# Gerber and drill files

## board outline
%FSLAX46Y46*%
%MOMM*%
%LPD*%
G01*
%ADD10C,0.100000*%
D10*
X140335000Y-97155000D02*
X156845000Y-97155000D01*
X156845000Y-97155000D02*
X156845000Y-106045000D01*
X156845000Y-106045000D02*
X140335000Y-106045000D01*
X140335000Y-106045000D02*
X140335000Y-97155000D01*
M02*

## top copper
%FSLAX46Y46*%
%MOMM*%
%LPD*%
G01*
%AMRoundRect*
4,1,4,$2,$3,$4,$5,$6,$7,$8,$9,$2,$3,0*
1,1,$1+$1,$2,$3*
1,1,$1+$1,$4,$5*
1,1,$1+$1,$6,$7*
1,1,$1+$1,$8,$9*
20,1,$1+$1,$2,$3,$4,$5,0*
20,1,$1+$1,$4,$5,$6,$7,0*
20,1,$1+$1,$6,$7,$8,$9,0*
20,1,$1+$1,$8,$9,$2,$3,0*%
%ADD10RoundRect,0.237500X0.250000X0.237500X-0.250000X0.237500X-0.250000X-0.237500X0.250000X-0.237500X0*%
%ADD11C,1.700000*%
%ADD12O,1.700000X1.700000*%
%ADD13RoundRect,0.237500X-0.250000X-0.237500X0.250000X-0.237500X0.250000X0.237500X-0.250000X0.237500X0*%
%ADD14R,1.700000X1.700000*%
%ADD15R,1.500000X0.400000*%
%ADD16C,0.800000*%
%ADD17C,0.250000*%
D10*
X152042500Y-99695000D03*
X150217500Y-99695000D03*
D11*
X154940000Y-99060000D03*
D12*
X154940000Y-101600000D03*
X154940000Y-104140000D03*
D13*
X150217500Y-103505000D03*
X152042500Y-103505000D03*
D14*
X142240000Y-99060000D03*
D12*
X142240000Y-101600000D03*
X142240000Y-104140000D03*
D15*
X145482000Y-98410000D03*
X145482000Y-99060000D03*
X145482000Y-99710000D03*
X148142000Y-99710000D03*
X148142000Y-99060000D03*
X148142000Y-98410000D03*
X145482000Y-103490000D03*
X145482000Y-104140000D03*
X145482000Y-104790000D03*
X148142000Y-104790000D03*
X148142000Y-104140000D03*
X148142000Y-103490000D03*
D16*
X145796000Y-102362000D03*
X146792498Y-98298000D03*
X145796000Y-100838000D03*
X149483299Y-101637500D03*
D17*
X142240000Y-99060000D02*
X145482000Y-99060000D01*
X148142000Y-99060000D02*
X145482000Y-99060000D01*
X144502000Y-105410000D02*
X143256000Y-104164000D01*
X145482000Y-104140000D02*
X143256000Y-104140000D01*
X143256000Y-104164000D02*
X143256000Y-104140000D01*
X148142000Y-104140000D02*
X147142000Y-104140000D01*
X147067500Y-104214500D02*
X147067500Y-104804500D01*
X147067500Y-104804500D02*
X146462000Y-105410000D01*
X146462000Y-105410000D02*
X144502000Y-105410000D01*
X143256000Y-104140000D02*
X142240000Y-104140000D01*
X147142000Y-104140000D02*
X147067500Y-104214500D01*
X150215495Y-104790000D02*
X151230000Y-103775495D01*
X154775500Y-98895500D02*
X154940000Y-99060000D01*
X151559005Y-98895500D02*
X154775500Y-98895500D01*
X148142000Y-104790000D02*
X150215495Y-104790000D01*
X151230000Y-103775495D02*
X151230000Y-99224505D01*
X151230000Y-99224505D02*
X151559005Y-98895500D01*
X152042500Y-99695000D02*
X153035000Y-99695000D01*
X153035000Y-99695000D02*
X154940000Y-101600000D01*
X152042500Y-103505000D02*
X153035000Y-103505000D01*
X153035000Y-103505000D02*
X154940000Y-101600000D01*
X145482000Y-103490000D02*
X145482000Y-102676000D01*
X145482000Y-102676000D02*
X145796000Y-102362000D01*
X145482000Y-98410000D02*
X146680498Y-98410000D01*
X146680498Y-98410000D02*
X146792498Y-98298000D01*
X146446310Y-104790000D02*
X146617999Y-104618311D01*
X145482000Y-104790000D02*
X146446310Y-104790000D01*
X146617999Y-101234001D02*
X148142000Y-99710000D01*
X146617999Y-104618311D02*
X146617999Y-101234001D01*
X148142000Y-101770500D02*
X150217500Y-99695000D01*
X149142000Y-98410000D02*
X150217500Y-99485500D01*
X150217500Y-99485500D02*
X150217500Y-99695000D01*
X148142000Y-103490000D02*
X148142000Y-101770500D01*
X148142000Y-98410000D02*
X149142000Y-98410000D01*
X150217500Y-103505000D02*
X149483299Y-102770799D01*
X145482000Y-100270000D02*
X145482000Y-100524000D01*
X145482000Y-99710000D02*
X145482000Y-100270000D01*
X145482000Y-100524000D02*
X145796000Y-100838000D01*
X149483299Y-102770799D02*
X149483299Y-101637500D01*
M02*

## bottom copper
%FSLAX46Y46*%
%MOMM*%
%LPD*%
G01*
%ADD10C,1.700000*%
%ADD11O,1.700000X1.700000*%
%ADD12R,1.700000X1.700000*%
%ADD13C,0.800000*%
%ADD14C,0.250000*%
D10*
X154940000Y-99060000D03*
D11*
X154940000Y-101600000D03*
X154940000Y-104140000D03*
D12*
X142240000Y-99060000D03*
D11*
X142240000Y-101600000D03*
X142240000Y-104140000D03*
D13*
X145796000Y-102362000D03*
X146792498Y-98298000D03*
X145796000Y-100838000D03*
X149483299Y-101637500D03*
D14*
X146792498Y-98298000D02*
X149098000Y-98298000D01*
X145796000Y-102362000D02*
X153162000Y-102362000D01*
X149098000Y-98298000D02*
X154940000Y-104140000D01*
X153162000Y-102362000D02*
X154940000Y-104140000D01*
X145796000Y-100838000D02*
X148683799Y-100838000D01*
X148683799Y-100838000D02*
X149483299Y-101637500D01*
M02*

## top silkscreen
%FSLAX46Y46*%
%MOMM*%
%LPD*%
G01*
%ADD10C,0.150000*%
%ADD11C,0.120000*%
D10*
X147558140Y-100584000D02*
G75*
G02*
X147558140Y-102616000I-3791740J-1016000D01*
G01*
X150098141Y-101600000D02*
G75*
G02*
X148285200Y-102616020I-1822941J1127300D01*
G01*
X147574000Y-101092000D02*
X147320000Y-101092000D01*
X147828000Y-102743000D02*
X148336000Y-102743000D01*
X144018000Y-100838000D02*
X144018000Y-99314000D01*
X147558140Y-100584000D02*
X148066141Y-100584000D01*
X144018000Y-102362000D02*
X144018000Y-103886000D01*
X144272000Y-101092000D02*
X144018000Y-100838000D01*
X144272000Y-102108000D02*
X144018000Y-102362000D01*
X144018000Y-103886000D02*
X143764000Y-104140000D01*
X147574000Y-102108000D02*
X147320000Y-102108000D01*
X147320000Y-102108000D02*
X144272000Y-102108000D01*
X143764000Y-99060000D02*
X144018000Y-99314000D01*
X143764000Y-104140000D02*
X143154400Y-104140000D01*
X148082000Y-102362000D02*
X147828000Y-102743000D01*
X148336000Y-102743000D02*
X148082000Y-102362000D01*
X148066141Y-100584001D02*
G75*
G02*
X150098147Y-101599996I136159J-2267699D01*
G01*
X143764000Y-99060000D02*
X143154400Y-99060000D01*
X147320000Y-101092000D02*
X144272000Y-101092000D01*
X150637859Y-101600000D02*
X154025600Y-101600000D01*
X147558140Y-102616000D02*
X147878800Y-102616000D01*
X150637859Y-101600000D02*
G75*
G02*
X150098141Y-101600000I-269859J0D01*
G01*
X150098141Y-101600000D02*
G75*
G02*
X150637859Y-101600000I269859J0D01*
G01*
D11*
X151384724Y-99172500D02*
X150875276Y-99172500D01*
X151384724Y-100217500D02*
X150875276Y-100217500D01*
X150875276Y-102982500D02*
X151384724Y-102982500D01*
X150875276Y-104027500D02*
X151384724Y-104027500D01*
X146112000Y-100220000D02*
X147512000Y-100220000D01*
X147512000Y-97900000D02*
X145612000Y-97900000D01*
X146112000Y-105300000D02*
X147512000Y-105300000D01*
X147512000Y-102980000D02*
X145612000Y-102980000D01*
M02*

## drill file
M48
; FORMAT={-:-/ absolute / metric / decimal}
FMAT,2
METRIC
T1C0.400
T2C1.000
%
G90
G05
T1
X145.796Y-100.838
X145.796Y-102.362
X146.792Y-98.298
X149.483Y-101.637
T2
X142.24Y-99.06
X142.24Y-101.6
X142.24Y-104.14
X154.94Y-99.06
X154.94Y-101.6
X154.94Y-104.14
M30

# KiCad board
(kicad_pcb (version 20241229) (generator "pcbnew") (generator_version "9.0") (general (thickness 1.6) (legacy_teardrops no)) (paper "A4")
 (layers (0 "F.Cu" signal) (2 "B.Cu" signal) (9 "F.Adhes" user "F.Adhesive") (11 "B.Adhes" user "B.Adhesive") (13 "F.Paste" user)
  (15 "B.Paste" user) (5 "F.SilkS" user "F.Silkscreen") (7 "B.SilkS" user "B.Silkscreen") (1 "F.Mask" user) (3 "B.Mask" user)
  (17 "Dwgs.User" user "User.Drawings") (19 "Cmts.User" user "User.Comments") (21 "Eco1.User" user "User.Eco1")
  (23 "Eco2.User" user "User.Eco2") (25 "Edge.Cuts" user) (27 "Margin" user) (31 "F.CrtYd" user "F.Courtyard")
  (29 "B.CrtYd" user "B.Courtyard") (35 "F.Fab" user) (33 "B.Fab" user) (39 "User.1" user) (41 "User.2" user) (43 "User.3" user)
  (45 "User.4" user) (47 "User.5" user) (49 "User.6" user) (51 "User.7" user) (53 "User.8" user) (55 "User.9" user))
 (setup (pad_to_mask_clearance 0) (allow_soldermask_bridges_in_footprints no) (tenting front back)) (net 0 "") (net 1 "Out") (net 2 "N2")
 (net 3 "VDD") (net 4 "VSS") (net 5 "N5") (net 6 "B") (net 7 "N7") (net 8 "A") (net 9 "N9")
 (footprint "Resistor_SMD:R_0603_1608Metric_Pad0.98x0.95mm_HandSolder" (layer "F.Cu") (at 151.13 99.695 180)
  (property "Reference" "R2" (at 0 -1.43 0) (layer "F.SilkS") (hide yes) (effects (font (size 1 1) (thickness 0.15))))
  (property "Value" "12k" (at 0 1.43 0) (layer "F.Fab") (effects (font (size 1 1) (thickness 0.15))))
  (fp_line (start -0.254724 0.5225) (end 0.254724 0.5225) (stroke (width 0.12) (type solid)) (layer "F.SilkS"))
  (fp_line (start -0.254724 -0.5225) (end 0.254724 -0.5225) (stroke (width 0.12) (type solid)) (layer "F.SilkS"))
  (pad "1" smd roundrect (at -0.9125 0 180) (size 0.975 0.95) (layers "F.Cu" "F.Mask" "F.Paste") (roundrect_rratio 0.25) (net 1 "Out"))
  (pad "2" smd roundrect (at 0.9125 0 180) (size 0.975 0.95) (layers "F.Cu" "F.Mask" "F.Paste") (roundrect_rratio 0.25) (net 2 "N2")))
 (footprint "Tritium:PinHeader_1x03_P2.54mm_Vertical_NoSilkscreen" (layer "F.Cu") (at 154.94 99.06)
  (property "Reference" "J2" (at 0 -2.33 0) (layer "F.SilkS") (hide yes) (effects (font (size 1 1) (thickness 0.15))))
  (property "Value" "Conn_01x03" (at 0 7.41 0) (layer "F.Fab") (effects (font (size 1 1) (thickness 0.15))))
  (pad "1" thru_hole circle (at 0 0) (size 1.7 1.7) (drill 1) (layers "*.Cu" "*.Mask") (remove_unused_layers no) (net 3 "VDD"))
  (pad "2" thru_hole oval (at 0 2.54) (size 1.7 1.7) (drill 1) (layers "*.Cu" "*.Mask") (remove_unused_layers no) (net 1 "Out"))
  (pad "3" thru_hole oval (at 0 5.08) (size 1.7 1.7) (drill 1) (layers "*.Cu" "*.Mask") (remove_unused_layers no) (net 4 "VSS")))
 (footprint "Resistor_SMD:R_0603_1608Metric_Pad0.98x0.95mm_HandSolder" (layer "F.Cu") (at 151.13 103.505)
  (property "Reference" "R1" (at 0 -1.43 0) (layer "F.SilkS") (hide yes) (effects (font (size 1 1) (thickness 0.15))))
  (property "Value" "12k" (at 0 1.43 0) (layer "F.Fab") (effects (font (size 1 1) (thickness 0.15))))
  (fp_line (start -0.254724 -0.5225) (end 0.254724 -0.5225) (stroke (width 0.12) (type solid)) (layer "F.SilkS"))
  (fp_line (start -0.254724 0.5225) (end 0.254724 0.5225) (stroke (width 0.12) (type solid)) (layer "F.SilkS"))
  (pad "1" smd roundrect (at -0.9125 0) (size 0.975 0.95) (layers "F.Cu" "F.Mask" "F.Paste") (roundrect_rratio 0.25) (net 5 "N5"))
  (pad "2" smd roundrect (at 0.9125 0) (size 0.975 0.95) (layers "F.Cu" "F.Mask" "F.Paste") (roundrect_rratio 0.25) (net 1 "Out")))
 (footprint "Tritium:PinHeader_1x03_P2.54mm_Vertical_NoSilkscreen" (layer "F.Cu") (at 142.24 99.06)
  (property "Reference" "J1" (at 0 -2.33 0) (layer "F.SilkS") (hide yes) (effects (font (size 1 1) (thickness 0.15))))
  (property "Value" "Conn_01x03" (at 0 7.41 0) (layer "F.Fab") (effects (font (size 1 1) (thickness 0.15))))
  (pad "1" thru_hole rect (at 0 0) (size 1.7 1.7) (drill 1) (layers "*.Cu" "*.Mask") (remove_unused_layers no) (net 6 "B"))
  (pad "2" thru_hole oval (at 0 2.54) (size 1.7 1.7) (drill 1) (layers "*.Cu" "*.Mask") (remove_unused_layers no) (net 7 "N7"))
  (pad "3" thru_hole oval (at 0 5.08) (size 1.7 1.7) (drill 1) (layers "*.Cu" "*.Mask") (remove_unused_layers no) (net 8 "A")))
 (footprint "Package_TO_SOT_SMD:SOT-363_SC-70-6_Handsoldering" (layer "F.Cu") (at 146.812 99.06)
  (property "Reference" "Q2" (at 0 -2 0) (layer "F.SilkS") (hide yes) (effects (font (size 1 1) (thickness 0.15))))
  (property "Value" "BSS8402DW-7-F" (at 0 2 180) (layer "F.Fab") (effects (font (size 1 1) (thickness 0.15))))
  (fp_line (start -0.7 1.16) (end 0.7 1.16) (stroke (width 0.12) (type solid)) (layer "F.SilkS"))
  (fp_line (start 0.7 -1.16) (end -1.2 -1.16) (stroke (width 0.12) (type solid)) (layer "F.SilkS"))
  (pad "1" smd rect (at -1.33 -0.65) (size 1.5 0.4) (layers "F.Cu" "F.Mask" "F.Paste") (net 4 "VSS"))
  (pad "2" smd rect (at -1.33 0) (size 1.5 0.4) (layers "F.Cu" "F.Mask" "F.Paste") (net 6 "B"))
  (pad "3" smd rect (at -1.33 0.65) (size 1.5 0.4) (layers "F.Cu" "F.Mask" "F.Paste") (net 5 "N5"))
  (pad "4" smd rect (at 1.33 0.65) (size 1.5 0.4) (layers "F.Cu" "F.Mask" "F.Paste") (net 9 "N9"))
  (pad "5" smd rect (at 1.33 0) (size 1.5 0.4) (layers "F.Cu" "F.Mask" "F.Paste") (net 6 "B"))
  (pad "6" smd rect (at 1.33 -0.65) (size 1.5 0.4) (layers "F.Cu" "F.Mask" "F.Paste") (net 2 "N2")))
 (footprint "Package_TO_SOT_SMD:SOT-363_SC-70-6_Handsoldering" (layer "F.Cu") (at 146.812 104.14)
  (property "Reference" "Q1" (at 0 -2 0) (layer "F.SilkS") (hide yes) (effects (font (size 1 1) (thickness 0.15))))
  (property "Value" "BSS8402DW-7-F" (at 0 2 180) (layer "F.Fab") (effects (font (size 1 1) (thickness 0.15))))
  (fp_line (start -0.7 1.16) (end 0.7 1.16) (stroke (width 0.12) (type solid)) (layer "F.SilkS"))
  (fp_line (start 0.7 -1.16) (end -1.2 -1.16) (stroke (width 0.12) (type solid)) (layer "F.SilkS"))
  (pad "1" smd rect (at -1.33 -0.65) (size 1.5 0.4) (layers "F.Cu" "F.Mask" "F.Paste") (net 4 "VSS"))
  (pad "2" smd rect (at -1.33 0) (size 1.5 0.4) (layers "F.Cu" "F.Mask" "F.Paste") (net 8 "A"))
  (pad "3" smd rect (at -1.33 0.65) (size 1.5 0.4) (layers "F.Cu" "F.Mask" "F.Paste") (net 9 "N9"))
  (pad "4" smd rect (at 1.33 0.65) (size 1.5 0.4) (layers "F.Cu" "F.Mask" "F.Paste") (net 3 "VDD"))
  (pad "5" smd rect (at 1.33 0) (size 1.5 0.4) (layers "F.Cu" "F.Mask" "F.Paste") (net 8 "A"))
  (pad "6" smd rect (at 1.33 -0.65) (size 1.5 0.4) (layers "F.Cu" "F.Mask" "F.Paste") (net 2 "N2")))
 (gr_arc (start 147.55814 100.584) (mid 147.6919 101.6) (end 147.55814 102.616) (stroke (width 0.15) (type solid)) (layer "F.SilkS"))
 (gr_arc (start 150.098141 101.6) (mid 149.323048 102.342429) (end 148.2852 102.616) (stroke (width 0.15) (type solid)) (layer "F.SilkS"))
 (gr_line (start 147.574 101.092) (end 147.32 101.092) (stroke (width 0.15) (type solid)) (layer "F.SilkS"))
 (gr_line (start 147.828 102.743) (end 148.336 102.743) (stroke (width 0.15) (type solid)) (layer "F.SilkS"))
 (gr_line (start 144.018 100.838) (end 144.018 99.314) (stroke (width 0.15) (type solid)) (layer "F.SilkS"))
 (gr_line (start 147.55814 100.584) (end 148.066141 100.584) (stroke (width 0.15) (type solid)) (layer "F.SilkS"))
 (gr_line (start 144.018 102.362) (end 144.018 103.886) (stroke (width 0.15) (type solid)) (layer "F.SilkS"))
 (gr_line (start 144.272 101.092) (end 144.018 100.838) (stroke (width 0.15) (type solid)) (layer "F.SilkS"))
 (gr_line (start 144.272 102.108) (end 144.018 102.362) (stroke (width 0.15) (type solid)) (layer "F.SilkS"))
 (gr_line (start 144.018 103.886) (end 143.764 104.14) (stroke (width 0.15) (type solid)) (layer "F.SilkS"))
 (gr_line (start 147.574 102.108) (end 147.32 102.108) (stroke (width 0.15) (type solid)) (layer "F.SilkS"))
 (gr_line (start 147.32 102.108) (end 144.272 102.108) (stroke (width 0.15) (type solid)) (layer "F.SilkS"))
 (gr_line (start 143.764 99.06) (end 144.018 99.314) (stroke (width 0.15) (type solid)) (layer "F.SilkS"))
 (gr_line (start 143.764 104.14) (end 143.1544 104.14) (stroke (width 0.15) (type solid)) (layer "F.SilkS"))
 (gr_line (start 148.082 102.362) (end 147.828 102.743) (stroke (width 0.15) (type solid)) (layer "F.SilkS"))
 (gr_line (start 148.336 102.743) (end 148.082 102.362) (stroke (width 0.15) (type solid)) (layer "F.SilkS"))
 (gr_arc (start 148.066141 100.584001) (mid 149.218261 100.819761) (end 150.098141 101.6) (stroke (width 0.15) (type solid))
  (layer "F.SilkS"))
 (gr_line (start 143.764 99.06) (end 143.1544 99.06) (stroke (width 0.15) (type solid)) (layer "F.SilkS"))
 (gr_line (start 147.32 101.092) (end 144.272 101.092) (stroke (width 0.15) (type solid)) (layer "F.SilkS"))
 (gr_line (start 150.637859 101.6) (end 154.0256 101.6) (stroke (width 0.15) (type solid)) (layer "F.SilkS"))
 (gr_line (start 147.55814 102.616) (end 147.8788 102.616) (stroke (width 0.15) (type solid)) (layer "F.SilkS"))
 (gr_circle (center 150.368 101.6) (end 150.098141 101.6) (stroke (width 0.15) (type solid)) (fill no) (layer "F.SilkS"))
 (gr_line (start 140.335 97.155) (end 156.845 97.155) (stroke (width 0.1) (type solid)) (layer "Edge.Cuts"))
 (gr_line (start 156.845 97.155) (end 156.845 106.045) (stroke (width 0.1) (type solid)) (layer "Edge.Cuts"))
 (gr_line (start 156.845 106.045) (end 140.335 106.045) (stroke (width 0.1) (type solid)) (layer "Edge.Cuts"))
 (gr_line (start 140.335 106.045) (end 140.335 97.155) (stroke (width 0.1) (type solid)) (layer "Edge.Cuts"))
 (segment (start 142.24 99.06) (end 145.482 99.06) (width 0.25) (layer "F.Cu") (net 6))
 (segment (start 148.142 99.06) (end 145.482 99.06) (width 0.25) (layer "F.Cu") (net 6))
 (segment (start 144.502 105.41) (end 143.256 104.164) (width 0.25) (layer "F.Cu") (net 8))
 (segment (start 145.482 104.14) (end 143.256 104.14) (width 0.25) (layer "F.Cu") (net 8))
 (segment (start 143.256 104.164) (end 143.256 104.14) (width 0.25) (layer "F.Cu") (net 8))
 (segment (start 148.142 104.14) (end 147.142 104.14) (width 0.25) (layer "F.Cu") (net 8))
 (segment (start 147.0675 104.2145) (end 147.0675 104.8045) (width 0.25) (layer "F.Cu") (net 8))
 (segment (start 147.0675 104.8045) (end 146.462 105.41) (width 0.25) (layer "F.Cu") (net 8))
 (segment (start 146.462 105.41) (end 144.502 105.41) (width 0.25) (layer "F.Cu") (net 8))
 (segment (start 143.256 104.14) (end 142.24 104.14) (width 0.25) (layer "F.Cu") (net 8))
 (segment (start 147.142 104.14) (end 147.0675 104.2145) (width 0.25) (layer "F.Cu") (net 8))
 (segment (start 150.215495 104.79) (end 151.23 103.775495) (width 0.25) (layer "F.Cu") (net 3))
 (segment (start 154.7755 98.8955) (end 154.94 99.06) (width 0.25) (layer "F.Cu") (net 3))
 (segment (start 151.559005 98.8955) (end 154.7755 98.8955) (width 0.25) (layer "F.Cu") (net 3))
 (segment (start 148.142 104.79) (end 150.215495 104.79) (width 0.25) (layer "F.Cu") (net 3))
 (segment (start 151.23 103.775495) (end 151.23 99.224505) (width 0.25) (layer "F.Cu") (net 3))
 (segment (start 151.23 99.224505) (end 151.559005 98.8955) (width 0.25) (layer "F.Cu") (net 3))
 (segment (start 152.0425 99.695) (end 153.035 99.695) (width 0.25) (layer "F.Cu") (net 1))
 (segment (start 153.035 99.695) (end 154.94 101.6) (width 0.25) (layer "F.Cu") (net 1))
 (segment (start 152.0425 103.505) (end 153.035 103.505) (width 0.25) (layer "F.Cu") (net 1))
 (segment (start 153.035 103.505) (end 154.94 101.6) (width 0.25) (layer "F.Cu") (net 1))
 (segment (start 145.482 103.49) (end 145.482 102.676) (width 0.25) (layer "F.Cu") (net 4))
 (segment (start 145.482 102.676) (end 145.796 102.362) (width 0.25) (layer "F.Cu") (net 4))
 (segment (start 145.482 98.41) (end 146.680498 98.41) (width 0.25) (layer "F.Cu") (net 4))
 (segment (start 146.680498 98.41) (end 146.792498 98.298) (width 0.25) (layer "F.Cu") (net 4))
 (via (at 145.796 102.362) (size 0.8) (drill 0.4) (layers "F.Cu" "B.Cu") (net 4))
 (via (at 146.792498 98.298) (size 0.8) (drill 0.4) (layers "F.Cu" "B.Cu") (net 4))
 (segment (start 146.792498 98.298) (end 149.098 98.298) (width 0.25) (layer "B.Cu") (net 4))
 (segment (start 145.796 102.362) (end 153.162 102.362) (width 0.25) (layer "B.Cu") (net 4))
 (segment (start 149.098 98.298) (end 154.94 104.14) (width 0.25) (layer "B.Cu") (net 4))
 (segment (start 153.162 102.362) (end 154.94 104.14) (width 0.25) (layer "B.Cu") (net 4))
 (segment (start 146.44631 104.79) (end 146.617999 104.618311) (width 0.25) (layer "F.Cu") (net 9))
 (segment (start 145.482 104.79) (end 146.44631 104.79) (width 0.25) (layer "F.Cu") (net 9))
 (segment (start 146.617999 101.234001) (end 148.142 99.71) (width 0.25) (layer "F.Cu") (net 9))
 (segment (start 146.617999 104.618311) (end 146.617999 101.234001) (width 0.25) (layer "F.Cu") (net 9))
 (segment (start 148.142 101.7705) (end 150.2175 99.695) (width 0.25) (layer "F.Cu") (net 2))
 (segment (start 149.142 98.41) (end 150.2175 99.4855) (width 0.25) (layer "F.Cu") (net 2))
 (segment (start 150.2175 99.4855) (end 150.2175 99.695) (width 0.25) (layer "F.Cu") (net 2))
 (segment (start 148.142 103.49) (end 148.142 101.7705) (width 0.25) (layer "F.Cu") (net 2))
 (segment (start 148.142 98.41) (end 149.142 98.41) (width 0.25) (layer "F.Cu") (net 2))
 (segment (start 150.2175 103.505) (end 149.483299 102.770799) (width 0.25) (layer "F.Cu") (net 5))
 (segment (start 145.482 100.27) (end 145.482 100.524) (width 0.25) (layer "F.Cu") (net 5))
 (segment (start 145.482 99.71) (end 145.482 100.27) (width 0.25) (layer "F.Cu") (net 5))
 (segment (start 145.482 100.524) (end 145.796 100.838) (width 0.25) (layer "F.Cu") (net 5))
 (segment (start 149.483299 102.770799) (end 149.483299 101.6375) (width 0.25) (layer "F.Cu") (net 5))
 (via (at 145.796 100.838) (size 0.8) (drill 0.4) (layers "F.Cu" "B.Cu") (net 5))
 (via (at 149.483299 101.6375) (size 0.8) (drill 0.4) (layers "F.Cu" "B.Cu") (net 5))
 (segment (start 145.796 100.838) (end 148.683799 100.838) (width 0.25) (layer "B.Cu") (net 5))
 (segment (start 148.683799 100.838) (end 149.483299 101.6375) (width 0.25) (layer "B.Cu") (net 5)))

